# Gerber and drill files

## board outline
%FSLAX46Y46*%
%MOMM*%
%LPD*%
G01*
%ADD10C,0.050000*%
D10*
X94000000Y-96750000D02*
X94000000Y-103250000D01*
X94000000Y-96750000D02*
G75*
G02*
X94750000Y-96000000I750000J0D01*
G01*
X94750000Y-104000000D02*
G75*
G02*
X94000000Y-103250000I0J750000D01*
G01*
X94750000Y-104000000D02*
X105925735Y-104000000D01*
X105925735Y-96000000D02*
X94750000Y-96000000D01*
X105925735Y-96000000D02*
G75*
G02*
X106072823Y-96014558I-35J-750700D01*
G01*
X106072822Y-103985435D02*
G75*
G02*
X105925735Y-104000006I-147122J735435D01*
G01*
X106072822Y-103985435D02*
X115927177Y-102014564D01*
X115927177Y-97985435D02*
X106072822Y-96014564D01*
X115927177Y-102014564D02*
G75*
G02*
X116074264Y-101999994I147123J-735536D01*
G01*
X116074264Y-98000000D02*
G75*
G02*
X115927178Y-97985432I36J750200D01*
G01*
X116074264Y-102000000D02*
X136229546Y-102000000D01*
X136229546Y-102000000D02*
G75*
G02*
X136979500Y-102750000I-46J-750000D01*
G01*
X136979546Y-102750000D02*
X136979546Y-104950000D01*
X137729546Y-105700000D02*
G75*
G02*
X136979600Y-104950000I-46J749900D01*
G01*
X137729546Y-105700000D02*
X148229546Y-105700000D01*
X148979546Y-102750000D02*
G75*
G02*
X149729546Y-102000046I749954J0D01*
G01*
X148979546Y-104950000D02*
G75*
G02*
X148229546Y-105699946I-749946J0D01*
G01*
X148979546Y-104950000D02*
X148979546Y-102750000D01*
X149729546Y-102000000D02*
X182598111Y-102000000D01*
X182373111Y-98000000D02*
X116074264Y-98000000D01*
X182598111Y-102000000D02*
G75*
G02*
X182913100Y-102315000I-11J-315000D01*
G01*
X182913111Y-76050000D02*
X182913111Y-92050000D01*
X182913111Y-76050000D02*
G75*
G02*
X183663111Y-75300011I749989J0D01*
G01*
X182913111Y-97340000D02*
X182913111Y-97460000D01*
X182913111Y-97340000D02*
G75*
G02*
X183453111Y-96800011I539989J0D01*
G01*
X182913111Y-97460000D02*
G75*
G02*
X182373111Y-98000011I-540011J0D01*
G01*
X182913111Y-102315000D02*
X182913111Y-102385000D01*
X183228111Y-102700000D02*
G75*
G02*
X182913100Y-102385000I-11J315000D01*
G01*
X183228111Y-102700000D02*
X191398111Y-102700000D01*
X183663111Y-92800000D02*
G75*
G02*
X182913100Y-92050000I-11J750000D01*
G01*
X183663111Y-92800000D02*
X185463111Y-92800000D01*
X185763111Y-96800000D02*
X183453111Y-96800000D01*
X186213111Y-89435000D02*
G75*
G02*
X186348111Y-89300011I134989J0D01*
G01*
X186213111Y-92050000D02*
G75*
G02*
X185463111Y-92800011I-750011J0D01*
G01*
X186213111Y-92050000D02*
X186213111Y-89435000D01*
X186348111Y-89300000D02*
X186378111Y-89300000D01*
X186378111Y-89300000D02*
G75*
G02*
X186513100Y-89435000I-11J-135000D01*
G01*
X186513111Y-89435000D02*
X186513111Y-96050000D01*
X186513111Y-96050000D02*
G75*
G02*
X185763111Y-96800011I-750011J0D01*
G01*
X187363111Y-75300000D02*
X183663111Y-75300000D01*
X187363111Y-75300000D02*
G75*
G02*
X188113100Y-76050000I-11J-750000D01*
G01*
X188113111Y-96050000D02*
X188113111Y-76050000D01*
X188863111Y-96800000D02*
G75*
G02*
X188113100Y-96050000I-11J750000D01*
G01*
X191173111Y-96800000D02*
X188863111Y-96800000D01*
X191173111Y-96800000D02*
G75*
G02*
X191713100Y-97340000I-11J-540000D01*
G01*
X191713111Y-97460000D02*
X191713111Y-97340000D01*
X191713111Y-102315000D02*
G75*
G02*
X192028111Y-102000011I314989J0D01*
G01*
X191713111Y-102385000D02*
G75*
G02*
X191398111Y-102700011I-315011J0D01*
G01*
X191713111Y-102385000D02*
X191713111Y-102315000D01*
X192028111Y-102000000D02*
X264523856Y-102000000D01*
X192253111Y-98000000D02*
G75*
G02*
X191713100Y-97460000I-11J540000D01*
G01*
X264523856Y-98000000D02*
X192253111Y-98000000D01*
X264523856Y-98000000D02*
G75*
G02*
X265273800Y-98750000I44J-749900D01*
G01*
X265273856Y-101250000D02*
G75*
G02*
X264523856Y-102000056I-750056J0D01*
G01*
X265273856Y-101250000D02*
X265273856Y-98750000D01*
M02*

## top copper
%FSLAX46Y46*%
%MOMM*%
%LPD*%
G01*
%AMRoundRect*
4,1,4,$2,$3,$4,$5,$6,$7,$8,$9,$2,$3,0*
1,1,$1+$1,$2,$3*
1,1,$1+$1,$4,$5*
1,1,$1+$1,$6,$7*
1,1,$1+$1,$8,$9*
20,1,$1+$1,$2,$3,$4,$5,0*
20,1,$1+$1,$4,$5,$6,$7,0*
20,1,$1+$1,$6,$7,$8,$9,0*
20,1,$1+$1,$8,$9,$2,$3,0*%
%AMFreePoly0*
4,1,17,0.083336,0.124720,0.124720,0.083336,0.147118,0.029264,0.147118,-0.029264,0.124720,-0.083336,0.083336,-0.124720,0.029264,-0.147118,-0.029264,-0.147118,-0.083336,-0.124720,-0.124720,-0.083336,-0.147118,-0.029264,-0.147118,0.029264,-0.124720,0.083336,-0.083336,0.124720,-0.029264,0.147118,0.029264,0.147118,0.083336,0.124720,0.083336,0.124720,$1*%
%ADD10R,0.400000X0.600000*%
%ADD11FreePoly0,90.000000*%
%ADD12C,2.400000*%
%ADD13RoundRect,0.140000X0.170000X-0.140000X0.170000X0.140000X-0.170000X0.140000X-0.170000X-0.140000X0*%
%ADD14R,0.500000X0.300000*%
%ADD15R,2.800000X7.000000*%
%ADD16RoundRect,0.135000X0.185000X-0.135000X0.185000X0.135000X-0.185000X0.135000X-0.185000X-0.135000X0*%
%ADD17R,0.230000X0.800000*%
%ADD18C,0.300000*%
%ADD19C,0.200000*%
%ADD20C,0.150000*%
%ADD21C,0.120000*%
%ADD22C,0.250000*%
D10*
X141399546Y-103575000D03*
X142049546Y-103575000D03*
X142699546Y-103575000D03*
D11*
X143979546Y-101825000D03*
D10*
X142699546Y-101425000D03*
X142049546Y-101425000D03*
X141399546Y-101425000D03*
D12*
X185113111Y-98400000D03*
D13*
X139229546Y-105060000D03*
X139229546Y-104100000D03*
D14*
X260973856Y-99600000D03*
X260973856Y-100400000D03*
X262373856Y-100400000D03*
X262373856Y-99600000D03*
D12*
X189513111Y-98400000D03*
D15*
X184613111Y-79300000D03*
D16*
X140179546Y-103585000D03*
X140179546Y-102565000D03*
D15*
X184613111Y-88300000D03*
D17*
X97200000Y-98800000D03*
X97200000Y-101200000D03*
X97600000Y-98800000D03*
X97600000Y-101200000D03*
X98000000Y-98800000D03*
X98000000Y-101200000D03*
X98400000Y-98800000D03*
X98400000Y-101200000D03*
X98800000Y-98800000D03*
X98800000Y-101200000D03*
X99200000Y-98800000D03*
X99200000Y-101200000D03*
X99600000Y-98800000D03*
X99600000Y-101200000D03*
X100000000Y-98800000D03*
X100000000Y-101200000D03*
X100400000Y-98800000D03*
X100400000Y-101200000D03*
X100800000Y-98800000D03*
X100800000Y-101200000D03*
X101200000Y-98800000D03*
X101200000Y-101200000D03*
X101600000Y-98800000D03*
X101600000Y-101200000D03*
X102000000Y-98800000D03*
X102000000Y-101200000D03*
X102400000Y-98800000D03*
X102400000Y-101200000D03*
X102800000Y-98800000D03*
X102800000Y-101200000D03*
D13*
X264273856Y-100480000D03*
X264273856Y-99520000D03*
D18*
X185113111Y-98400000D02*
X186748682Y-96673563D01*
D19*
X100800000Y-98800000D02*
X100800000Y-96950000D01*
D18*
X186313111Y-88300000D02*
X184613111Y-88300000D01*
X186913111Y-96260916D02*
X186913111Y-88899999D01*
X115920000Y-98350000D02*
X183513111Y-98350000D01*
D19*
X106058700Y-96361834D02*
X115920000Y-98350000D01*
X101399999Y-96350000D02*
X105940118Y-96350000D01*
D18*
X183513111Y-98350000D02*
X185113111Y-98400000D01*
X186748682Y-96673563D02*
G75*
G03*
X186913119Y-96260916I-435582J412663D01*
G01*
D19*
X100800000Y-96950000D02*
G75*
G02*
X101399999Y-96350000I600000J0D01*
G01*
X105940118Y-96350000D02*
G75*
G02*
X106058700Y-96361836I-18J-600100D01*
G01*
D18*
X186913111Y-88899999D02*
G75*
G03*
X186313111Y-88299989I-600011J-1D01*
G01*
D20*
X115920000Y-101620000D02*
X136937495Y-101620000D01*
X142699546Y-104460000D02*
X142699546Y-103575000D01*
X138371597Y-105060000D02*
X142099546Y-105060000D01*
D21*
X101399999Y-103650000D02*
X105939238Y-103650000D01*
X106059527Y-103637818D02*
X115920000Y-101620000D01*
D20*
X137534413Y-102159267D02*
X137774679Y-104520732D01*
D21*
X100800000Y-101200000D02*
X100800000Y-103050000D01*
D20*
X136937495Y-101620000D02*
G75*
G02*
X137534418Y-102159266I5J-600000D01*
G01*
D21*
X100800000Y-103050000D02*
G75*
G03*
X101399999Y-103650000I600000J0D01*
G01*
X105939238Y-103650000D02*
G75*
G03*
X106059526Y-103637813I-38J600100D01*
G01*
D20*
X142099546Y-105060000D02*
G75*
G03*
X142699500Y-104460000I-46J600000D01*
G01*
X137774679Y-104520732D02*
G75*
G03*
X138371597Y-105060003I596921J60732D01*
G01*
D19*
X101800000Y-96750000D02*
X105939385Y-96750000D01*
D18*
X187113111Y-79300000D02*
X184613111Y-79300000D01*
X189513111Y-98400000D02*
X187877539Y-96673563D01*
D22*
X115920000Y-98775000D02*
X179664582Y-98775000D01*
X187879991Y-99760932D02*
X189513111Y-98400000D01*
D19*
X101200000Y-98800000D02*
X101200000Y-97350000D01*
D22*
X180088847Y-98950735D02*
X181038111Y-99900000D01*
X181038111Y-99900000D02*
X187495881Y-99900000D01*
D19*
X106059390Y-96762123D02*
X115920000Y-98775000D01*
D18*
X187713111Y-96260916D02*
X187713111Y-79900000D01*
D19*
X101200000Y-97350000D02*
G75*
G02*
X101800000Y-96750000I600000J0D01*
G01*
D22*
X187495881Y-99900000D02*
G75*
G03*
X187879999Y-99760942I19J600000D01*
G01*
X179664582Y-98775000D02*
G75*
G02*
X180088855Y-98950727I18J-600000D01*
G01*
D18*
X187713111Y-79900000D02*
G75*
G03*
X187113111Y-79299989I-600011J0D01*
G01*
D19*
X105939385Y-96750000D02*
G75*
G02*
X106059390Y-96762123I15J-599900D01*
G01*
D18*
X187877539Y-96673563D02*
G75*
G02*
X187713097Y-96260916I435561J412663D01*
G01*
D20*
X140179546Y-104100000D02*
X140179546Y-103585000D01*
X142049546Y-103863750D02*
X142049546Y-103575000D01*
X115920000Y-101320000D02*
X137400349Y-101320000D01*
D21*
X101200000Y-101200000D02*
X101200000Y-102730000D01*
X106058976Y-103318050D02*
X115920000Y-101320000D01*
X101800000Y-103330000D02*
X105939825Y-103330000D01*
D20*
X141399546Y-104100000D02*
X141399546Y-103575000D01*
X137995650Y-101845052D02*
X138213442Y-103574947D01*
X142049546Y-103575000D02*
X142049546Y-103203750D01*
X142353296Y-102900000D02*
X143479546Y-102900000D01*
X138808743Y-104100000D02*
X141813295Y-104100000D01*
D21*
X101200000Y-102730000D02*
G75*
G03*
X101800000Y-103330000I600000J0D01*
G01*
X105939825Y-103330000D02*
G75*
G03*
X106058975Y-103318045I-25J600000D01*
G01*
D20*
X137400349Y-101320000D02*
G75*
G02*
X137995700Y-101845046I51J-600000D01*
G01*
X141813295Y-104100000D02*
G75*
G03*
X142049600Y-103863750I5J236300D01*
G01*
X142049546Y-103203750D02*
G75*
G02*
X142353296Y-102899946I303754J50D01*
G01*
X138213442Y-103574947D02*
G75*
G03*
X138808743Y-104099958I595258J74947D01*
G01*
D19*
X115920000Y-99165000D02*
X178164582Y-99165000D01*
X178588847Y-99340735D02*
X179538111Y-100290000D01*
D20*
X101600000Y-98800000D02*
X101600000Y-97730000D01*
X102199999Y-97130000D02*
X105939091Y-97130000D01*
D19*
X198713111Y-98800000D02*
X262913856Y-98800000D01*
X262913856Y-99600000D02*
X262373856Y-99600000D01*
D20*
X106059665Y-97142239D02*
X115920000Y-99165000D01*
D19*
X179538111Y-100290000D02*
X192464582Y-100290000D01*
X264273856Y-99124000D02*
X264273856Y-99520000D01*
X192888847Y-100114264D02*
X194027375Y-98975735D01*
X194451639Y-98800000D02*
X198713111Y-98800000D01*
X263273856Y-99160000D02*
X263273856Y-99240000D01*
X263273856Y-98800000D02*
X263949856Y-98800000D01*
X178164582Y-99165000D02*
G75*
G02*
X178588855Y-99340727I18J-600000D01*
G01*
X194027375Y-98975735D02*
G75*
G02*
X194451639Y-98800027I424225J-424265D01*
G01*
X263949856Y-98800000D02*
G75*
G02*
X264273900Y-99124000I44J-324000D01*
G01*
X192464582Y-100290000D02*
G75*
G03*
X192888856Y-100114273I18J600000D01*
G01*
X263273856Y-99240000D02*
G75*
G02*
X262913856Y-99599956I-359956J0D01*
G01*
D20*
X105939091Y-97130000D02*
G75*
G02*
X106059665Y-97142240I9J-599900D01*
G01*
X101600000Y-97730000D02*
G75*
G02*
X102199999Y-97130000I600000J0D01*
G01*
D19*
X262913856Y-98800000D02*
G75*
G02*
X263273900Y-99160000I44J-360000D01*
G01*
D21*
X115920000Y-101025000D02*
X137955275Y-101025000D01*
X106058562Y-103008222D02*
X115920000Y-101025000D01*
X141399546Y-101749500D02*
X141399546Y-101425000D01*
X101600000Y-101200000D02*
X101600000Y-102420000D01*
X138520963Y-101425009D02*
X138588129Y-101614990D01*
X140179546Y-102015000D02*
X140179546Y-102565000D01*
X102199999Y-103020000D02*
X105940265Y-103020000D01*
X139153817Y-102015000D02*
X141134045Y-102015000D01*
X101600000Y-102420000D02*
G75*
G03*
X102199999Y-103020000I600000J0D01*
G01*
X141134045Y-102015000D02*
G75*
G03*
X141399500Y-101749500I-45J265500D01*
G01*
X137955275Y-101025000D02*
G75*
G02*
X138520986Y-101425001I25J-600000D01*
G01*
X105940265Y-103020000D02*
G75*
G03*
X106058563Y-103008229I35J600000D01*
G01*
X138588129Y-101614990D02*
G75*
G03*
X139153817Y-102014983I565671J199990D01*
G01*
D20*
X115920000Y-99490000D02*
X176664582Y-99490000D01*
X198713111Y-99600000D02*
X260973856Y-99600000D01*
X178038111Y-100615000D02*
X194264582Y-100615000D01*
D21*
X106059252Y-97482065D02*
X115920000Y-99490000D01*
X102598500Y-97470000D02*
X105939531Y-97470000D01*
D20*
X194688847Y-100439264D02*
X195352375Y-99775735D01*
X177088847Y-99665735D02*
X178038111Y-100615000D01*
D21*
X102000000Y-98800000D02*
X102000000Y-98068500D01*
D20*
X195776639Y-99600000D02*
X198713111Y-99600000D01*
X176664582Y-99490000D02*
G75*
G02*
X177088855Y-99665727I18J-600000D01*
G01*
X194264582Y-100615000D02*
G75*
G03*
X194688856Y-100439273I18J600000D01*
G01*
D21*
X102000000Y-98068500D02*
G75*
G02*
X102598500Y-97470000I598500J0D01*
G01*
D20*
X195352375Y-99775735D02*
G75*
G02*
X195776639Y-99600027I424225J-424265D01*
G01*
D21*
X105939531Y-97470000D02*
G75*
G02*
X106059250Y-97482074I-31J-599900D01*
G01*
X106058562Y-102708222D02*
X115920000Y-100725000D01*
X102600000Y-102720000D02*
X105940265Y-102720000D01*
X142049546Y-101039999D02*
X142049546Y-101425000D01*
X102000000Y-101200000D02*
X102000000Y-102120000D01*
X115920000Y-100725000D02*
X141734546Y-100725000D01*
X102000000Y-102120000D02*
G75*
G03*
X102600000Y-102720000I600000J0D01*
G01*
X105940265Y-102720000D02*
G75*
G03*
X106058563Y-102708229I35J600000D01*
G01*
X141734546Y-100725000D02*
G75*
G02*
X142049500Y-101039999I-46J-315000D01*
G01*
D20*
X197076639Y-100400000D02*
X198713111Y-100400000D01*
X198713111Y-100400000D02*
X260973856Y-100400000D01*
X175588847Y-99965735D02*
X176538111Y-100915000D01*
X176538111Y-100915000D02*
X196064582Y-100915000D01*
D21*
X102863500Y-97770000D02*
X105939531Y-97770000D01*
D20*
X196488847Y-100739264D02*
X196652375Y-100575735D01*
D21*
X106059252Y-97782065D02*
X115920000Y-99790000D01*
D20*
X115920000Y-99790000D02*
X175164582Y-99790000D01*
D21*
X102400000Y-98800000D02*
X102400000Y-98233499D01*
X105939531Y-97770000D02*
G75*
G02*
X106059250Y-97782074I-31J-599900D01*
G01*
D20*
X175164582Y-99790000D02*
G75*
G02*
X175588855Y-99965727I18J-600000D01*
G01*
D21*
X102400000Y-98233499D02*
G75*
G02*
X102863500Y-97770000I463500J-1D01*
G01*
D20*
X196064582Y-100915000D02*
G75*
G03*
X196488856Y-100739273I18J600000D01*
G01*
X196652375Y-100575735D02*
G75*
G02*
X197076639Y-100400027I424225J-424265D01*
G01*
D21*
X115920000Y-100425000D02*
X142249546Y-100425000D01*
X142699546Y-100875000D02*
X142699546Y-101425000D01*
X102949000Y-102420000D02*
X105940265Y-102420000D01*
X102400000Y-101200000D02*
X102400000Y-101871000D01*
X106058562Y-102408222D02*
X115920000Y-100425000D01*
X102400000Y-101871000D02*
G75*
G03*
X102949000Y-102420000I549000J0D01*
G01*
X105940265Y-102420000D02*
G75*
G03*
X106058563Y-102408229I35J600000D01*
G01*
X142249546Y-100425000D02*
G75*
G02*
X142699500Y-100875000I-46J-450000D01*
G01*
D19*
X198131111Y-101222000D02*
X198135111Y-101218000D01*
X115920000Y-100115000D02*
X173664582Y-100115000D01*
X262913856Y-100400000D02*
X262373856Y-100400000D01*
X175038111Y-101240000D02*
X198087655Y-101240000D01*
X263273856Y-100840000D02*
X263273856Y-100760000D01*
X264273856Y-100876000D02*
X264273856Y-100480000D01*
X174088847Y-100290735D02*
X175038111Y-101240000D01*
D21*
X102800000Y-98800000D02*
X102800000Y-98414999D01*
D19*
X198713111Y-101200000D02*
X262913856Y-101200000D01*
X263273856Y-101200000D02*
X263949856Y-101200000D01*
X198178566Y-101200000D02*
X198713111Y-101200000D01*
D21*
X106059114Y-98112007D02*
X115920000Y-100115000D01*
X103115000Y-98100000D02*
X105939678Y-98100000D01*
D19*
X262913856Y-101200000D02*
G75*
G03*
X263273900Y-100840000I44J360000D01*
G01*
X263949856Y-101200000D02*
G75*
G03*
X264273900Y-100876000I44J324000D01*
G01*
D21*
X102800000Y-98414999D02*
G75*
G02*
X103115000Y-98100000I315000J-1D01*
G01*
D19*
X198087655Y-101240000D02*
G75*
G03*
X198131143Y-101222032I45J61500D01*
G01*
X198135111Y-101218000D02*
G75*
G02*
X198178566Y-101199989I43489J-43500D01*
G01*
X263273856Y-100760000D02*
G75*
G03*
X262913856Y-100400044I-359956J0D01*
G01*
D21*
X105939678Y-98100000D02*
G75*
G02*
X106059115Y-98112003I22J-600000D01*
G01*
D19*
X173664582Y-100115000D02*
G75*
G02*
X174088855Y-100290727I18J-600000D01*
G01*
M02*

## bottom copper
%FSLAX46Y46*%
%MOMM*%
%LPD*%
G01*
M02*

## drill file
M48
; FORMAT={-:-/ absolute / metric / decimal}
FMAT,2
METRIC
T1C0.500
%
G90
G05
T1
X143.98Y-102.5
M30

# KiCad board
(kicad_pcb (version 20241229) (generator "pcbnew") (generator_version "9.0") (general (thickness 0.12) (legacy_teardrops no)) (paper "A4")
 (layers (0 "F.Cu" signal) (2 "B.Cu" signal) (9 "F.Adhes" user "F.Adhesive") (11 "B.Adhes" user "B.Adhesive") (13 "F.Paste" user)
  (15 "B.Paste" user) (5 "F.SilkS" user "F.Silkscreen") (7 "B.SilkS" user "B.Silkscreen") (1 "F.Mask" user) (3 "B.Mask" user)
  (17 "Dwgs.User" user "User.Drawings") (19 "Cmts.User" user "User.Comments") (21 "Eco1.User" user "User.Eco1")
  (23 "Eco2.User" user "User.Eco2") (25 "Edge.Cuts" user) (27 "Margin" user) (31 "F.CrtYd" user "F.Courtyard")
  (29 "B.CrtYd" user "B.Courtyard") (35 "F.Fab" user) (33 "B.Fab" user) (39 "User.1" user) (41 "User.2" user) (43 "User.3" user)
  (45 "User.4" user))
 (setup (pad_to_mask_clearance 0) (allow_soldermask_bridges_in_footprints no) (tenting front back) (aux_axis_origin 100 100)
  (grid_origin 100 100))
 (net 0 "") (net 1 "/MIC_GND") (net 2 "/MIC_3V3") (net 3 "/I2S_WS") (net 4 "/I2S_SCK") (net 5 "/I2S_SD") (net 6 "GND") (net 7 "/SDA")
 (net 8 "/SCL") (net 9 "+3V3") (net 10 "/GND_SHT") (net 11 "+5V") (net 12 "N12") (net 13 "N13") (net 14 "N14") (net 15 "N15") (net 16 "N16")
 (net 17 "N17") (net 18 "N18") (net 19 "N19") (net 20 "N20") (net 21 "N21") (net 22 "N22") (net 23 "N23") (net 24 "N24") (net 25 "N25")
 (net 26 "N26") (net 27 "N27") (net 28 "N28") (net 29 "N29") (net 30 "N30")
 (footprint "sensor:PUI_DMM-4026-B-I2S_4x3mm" (layer "F.Cu") (at 142.979546 102.5 90)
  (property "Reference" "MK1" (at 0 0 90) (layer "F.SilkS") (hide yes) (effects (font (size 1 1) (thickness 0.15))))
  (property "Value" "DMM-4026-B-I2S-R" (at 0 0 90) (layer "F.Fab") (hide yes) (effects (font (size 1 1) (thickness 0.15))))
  (pad "" np_thru_hole circle (at 0 1 90) (size 0.5 0.5) (drill 0.5) (layers "*.Mask"))
  (pad "1" smd rect (at -1.075 -1.58 90) (size 0.6 0.4) (layers "F.Cu" "F.Mask" "F.Paste") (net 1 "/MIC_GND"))
  (pad "2" smd rect (at -1.075 -0.93 90) (size 0.6 0.4) (layers "F.Cu" "F.Mask" "F.Paste") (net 1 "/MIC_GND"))
  (pad "3" smd rect (at -1.075 -0.28 90) (size 0.6 0.4) (layers "F.Cu" "F.Mask" "F.Paste") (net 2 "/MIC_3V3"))
  (pad "4" smd custom (at 0.675 1 90) (size 0.3 0.3) (layers "F.Cu" "F.Mask" "F.Paste") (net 1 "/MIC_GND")
   (options (clearance outline) (anchor circle)) (primitives))
  (pad "5" smd rect (at 1.075 -0.28 90) (size 0.6 0.4) (layers "F.Cu" "F.Mask" "F.Paste") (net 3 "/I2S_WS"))
  (pad "6" smd rect (at 1.075 -0.93 90) (size 0.6 0.4) (layers "F.Cu" "F.Mask" "F.Paste") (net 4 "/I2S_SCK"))
  (pad "7" smd rect (at 1.075 -1.58 90) (size 0.6 0.4) (layers "F.Cu" "F.Mask" "F.Paste") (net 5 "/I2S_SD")))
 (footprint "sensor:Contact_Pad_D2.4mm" (layer "F.Cu") (at 185.113111 98.4)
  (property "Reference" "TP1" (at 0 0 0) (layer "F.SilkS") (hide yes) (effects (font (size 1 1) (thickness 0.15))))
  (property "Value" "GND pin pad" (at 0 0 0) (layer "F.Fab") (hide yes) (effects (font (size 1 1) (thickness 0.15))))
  (pad "1" smd circle (at 0 0) (size 2.4 2.4) (layers "F.Cu" "F.Mask") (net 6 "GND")))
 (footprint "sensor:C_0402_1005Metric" (layer "F.Cu") (at 139.229546 104.58 90)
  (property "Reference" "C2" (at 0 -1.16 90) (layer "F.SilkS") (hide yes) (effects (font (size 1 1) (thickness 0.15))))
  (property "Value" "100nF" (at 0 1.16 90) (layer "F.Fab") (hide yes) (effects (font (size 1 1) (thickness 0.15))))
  (pad "1" smd roundrect (at -0.48 0 90) (size 0.56 0.62) (layers "F.Cu" "F.Mask" "F.Paste") (roundrect_rratio 0.25) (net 2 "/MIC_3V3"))
  (pad "2" smd roundrect (at 0.48 0 90) (size 0.56 0.62) (layers "F.Cu" "F.Mask" "F.Paste") (roundrect_rratio 0.25) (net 1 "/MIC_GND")))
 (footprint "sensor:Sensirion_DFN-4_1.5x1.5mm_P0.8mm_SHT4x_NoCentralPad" (layer "F.Cu") (at 261.673856 100)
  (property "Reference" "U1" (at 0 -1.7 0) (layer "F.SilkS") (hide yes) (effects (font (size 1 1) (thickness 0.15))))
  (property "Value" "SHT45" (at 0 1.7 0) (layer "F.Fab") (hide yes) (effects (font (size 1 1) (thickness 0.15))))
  (pad "1" smd rect (at -0.7 -0.4) (size 0.5 0.3) (layers "F.Cu" "F.Mask" "F.Paste") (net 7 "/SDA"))
  (pad "2" smd rect (at -0.7 0.4) (size 0.5 0.3) (layers "F.Cu" "F.Mask" "F.Paste") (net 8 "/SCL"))
  (pad "3" smd rect (at 0.7 0.4) (size 0.5 0.3) (layers "F.Cu" "F.Mask" "F.Paste") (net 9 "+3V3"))
  (pad "4" smd rect (at 0.7 -0.4) (size 0.5 0.3) (layers "F.Cu" "F.Mask" "F.Paste") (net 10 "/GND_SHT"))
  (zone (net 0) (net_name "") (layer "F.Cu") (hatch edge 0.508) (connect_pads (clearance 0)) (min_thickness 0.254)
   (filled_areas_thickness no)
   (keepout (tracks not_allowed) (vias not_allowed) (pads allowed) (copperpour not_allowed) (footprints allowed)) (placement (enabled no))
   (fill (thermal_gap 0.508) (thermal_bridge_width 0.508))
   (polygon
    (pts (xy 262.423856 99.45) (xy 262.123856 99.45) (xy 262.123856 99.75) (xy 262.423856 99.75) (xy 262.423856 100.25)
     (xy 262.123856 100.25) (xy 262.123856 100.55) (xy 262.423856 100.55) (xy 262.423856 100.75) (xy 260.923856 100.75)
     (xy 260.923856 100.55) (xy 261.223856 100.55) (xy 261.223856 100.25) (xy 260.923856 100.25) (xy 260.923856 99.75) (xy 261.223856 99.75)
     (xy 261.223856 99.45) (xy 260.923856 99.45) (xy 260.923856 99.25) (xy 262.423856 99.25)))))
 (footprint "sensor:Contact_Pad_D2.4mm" (layer "F.Cu") (at 189.513111 98.4)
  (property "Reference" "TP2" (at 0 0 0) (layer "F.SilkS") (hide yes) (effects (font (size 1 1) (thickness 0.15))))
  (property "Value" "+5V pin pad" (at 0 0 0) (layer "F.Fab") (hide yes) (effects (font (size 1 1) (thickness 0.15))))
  (pad "1" smd circle (at 0 0) (size 2.4 2.4) (layers "F.Cu" "F.Mask") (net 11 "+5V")))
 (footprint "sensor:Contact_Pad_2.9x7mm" (layer "F.Cu") (at 184.613111 79.3)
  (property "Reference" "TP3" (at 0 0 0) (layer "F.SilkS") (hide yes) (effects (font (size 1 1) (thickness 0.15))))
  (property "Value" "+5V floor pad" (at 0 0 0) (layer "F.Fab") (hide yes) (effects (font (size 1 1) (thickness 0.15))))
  (pad "1" smd rect (at 0 0) (size 2.8 7) (layers "F.Cu" "F.Mask") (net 11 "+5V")))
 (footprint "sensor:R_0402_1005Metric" (layer "F.Cu") (at 140.179546 103.075 90)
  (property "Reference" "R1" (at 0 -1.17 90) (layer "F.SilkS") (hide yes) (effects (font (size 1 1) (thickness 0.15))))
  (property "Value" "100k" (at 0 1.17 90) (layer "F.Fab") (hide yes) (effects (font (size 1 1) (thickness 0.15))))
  (pad "1" smd roundrect (at -0.51 0 90) (size 0.54 0.64) (layers "F.Cu" "F.Mask" "F.Paste") (roundrect_rratio 0.25) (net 1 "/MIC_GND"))
  (pad "2" smd roundrect (at 0.51 0 90) (size 0.54 0.64) (layers "F.Cu" "F.Mask" "F.Paste") (roundrect_rratio 0.25) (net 5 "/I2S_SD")))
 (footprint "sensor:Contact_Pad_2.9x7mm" (layer "F.Cu") (at 184.613111 88.3)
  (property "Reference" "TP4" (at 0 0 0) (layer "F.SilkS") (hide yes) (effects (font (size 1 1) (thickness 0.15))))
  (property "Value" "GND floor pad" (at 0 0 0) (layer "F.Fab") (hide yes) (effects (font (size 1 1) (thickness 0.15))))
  (pad "1" smd rect (at 0 0) (size 2.8 7) (layers "F.Cu" "F.Mask") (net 6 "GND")))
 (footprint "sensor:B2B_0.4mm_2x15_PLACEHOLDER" (layer "F.Cu") (at 100 100)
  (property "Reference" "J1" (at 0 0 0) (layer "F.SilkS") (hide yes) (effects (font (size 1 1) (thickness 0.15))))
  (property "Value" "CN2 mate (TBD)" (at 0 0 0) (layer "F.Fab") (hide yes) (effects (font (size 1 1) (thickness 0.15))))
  (pad "1" smd rect (at -2.8 -1.2) (size 0.23 0.8) (layers "F.Cu" "F.Mask" "F.Paste") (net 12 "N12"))
  (pad "2" smd rect (at -2.8 1.2) (size 0.23 0.8) (layers "F.Cu" "F.Mask" "F.Paste") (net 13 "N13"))
  (pad "3" smd rect (at -2.4 -1.2) (size 0.23 0.8) (layers "F.Cu" "F.Mask" "F.Paste") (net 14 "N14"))
  (pad "4" smd rect (at -2.4 1.2) (size 0.23 0.8) (layers "F.Cu" "F.Mask" "F.Paste") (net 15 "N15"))
  (pad "5" smd rect (at -2 -1.2) (size 0.23 0.8) (layers "F.Cu" "F.Mask" "F.Paste") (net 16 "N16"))
  (pad "6" smd rect (at -2 1.2) (size 0.23 0.8) (layers "F.Cu" "F.Mask" "F.Paste") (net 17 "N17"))
  (pad "7" smd rect (at -1.6 -1.2) (size 0.23 0.8) (layers "F.Cu" "F.Mask" "F.Paste") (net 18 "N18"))
  (pad "8" smd rect (at -1.6 1.2) (size 0.23 0.8) (layers "F.Cu" "F.Mask" "F.Paste") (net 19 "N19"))
  (pad "9" smd rect (at -1.2 -1.2) (size 0.23 0.8) (layers "F.Cu" "F.Mask" "F.Paste") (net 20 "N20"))
  (pad "10" smd rect (at -1.2 1.2) (size 0.23 0.8) (layers "F.Cu" "F.Mask" "F.Paste") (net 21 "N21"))
  (pad "11" smd rect (at -0.8 -1.2) (size 0.23 0.8) (layers "F.Cu" "F.Mask" "F.Paste") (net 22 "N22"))
  (pad "12" smd rect (at -0.8 1.2) (size 0.23 0.8) (layers "F.Cu" "F.Mask" "F.Paste") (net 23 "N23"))
  (pad "13" smd rect (at -0.4 -1.2) (size 0.23 0.8) (layers "F.Cu" "F.Mask" "F.Paste") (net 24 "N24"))
  (pad "14" smd rect (at -0.4 1.2) (size 0.23 0.8) (layers "F.Cu" "F.Mask" "F.Paste") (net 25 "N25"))
  (pad "15" smd rect (at 0 -1.2) (size 0.23 0.8) (layers "F.Cu" "F.Mask" "F.Paste") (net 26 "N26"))
  (pad "16" smd rect (at 0 1.2) (size 0.23 0.8) (layers "F.Cu" "F.Mask" "F.Paste") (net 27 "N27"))
  (pad "17" smd rect (at 0.4 -1.2) (size 0.23 0.8) (layers "F.Cu" "F.Mask" "F.Paste") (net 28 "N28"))
  (pad "18" smd rect (at 0.4 1.2) (size 0.23 0.8) (layers "F.Cu" "F.Mask" "F.Paste") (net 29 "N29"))
  (pad "19" smd rect (at 0.8 -1.2) (size 0.23 0.8) (layers "F.Cu" "F.Mask" "F.Paste") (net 6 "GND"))
  (pad "20" smd rect (at 0.8 1.2) (size 0.23 0.8) (layers "F.Cu" "F.Mask" "F.Paste") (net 2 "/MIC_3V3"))
  (pad "21" smd rect (at 1.2 -1.2) (size 0.23 0.8) (layers "F.Cu" "F.Mask" "F.Paste") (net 11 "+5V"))
  (pad "22" smd rect (at 1.2 1.2) (size 0.23 0.8) (layers "F.Cu" "F.Mask" "F.Paste") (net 1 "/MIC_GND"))
  (pad "23" smd rect (at 1.6 -1.2) (size 0.23 0.8) (layers "F.Cu" "F.Mask" "F.Paste") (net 10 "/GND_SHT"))
  (pad "24" smd rect (at 1.6 1.2) (size 0.23 0.8) (layers "F.Cu" "F.Mask" "F.Paste") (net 5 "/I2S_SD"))
  (pad "25" smd rect (at 2 -1.2) (size 0.23 0.8) (layers "F.Cu" "F.Mask" "F.Paste") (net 7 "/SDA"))
  (pad "26" smd rect (at 2 1.2) (size 0.23 0.8) (layers "F.Cu" "F.Mask" "F.Paste") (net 4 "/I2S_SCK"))
  (pad "27" smd rect (at 2.4 -1.2) (size 0.23 0.8) (layers "F.Cu" "F.Mask" "F.Paste") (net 8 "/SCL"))
  (pad "28" smd rect (at 2.4 1.2) (size 0.23 0.8) (layers "F.Cu" "F.Mask" "F.Paste") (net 3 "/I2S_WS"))
  (pad "29" smd rect (at 2.8 -1.2) (size 0.23 0.8) (layers "F.Cu" "F.Mask" "F.Paste") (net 9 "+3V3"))
  (pad "30" smd rect (at 2.8 1.2) (size 0.23 0.8) (layers "F.Cu" "F.Mask" "F.Paste") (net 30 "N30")))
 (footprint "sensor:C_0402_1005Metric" (layer "F.Cu") (at 264.273856 100 90)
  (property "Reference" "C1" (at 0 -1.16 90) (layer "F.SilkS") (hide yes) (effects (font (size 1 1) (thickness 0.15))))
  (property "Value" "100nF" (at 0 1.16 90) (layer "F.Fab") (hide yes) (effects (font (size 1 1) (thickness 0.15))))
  (pad "1" smd roundrect (at -0.48 0 90) (size 0.56 0.62) (layers "F.Cu" "F.Mask" "F.Paste") (roundrect_rratio 0.25) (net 9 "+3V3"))
  (pad "2" smd roundrect (at 0.48 0 90) (size 0.56 0.62) (layers "F.Cu" "F.Mask" "F.Paste") (roundrect_rratio 0.25) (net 10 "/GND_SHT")))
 (gr_line (start 94 96.75) (end 94 103.25) (stroke (width 0.05) (type default)) (layer "Edge.Cuts"))
 (gr_arc (start 94 96.75) (mid 94.21967 96.21967) (end 94.75 96) (stroke (width 0.05) (type default)) (layer "Edge.Cuts"))
 (gr_arc (start 94.75 104) (mid 94.21967 103.78033) (end 94 103.25) (stroke (width 0.05) (type default)) (layer "Edge.Cuts"))
 (gr_line (start 94.75 104) (end 105.925735 104) (stroke (width 0.05) (type default)) (layer "Edge.Cuts"))
 (gr_line (start 105.925735 96) (end 94.75 96) (stroke (width 0.05) (type default)) (layer "Edge.Cuts"))
 (gr_arc (start 105.925735 96) (mid 105.999638 96.003653) (end 106.072822 96.014564) (stroke (width 0.05) (type default))
  (layer "Edge.Cuts"))
 (gr_arc (start 106.072822 103.985435) (mid 105.999638 103.99635) (end 105.925735 104) (stroke (width 0.05) (type default))
  (layer "Edge.Cuts"))
 (gr_line (start 106.072822 103.985435) (end 115.927177 102.014564) (stroke (width 0.05) (type default)) (layer "Edge.Cuts"))
 (gr_line (start 115.927177 97.985435) (end 106.072822 96.014564) (stroke (width 0.05) (type default)) (layer "Edge.Cuts"))
 (gr_arc (start 115.927177 102.014564) (mid 116.000361 102.00365) (end 116.074264 102) (stroke (width 0.05) (type default))
  (layer "Edge.Cuts"))
 (gr_arc (start 116.074264 98) (mid 116.000361 97.996349) (end 115.927177 97.985435) (stroke (width 0.05) (type default))
  (layer "Edge.Cuts"))
 (gr_line (start 116.074264 102) (end 136.229546 102) (stroke (width 0.05) (type default)) (layer "Edge.Cuts"))
 (gr_arc (start 136.229546 102) (mid 136.759876 102.219669) (end 136.979546 102.75) (stroke (width 0.05) (type default)) (layer "Edge.Cuts"))
 (gr_line (start 136.979546 102.75) (end 136.979546 104.95) (stroke (width 0.05) (type default)) (layer "Edge.Cuts"))
 (gr_arc (start 137.729546 105.7) (mid 137.199186 105.480346) (end 136.979546 104.95) (stroke (width 0.05) (type default))
  (layer "Edge.Cuts"))
 (gr_line (start 137.729546 105.7) (end 148.229546 105.7) (stroke (width 0.05) (type default)) (layer "Edge.Cuts"))
 (gr_arc (start 148.979546 102.75) (mid 149.199216 102.219669) (end 149.729546 102) (stroke (width 0.05) (type default)) (layer "Edge.Cuts"))
 (gr_arc (start 148.979546 104.95) (mid 148.759879 105.480346) (end 148.229546 105.7) (stroke (width 0.05) (type default))
  (layer "Edge.Cuts"))
 (gr_line (start 148.979546 104.95) (end 148.979546 102.75) (stroke (width 0.05) (type default)) (layer "Edge.Cuts"))
 (gr_line (start 149.729546 102) (end 182.598111 102) (stroke (width 0.05) (type default)) (layer "Edge.Cuts"))
 (gr_line (start 182.373111 98) (end 116.074264 98) (stroke (width 0.05) (type default)) (layer "Edge.Cuts"))
 (gr_arc (start 182.598111 102) (mid 182.820849 102.092261) (end 182.913111 102.315) (stroke (width 0.05) (type default))
  (layer "Edge.Cuts"))
 (gr_line (start 182.913111 76.05) (end 182.913111 92.05) (stroke (width 0.05) (type default)) (layer "Edge.Cuts"))
 (gr_arc (start 182.913111 76.05) (mid 183.132782 75.519674) (end 183.663111 75.3) (stroke (width 0.05) (type default)) (layer "Edge.Cuts"))
 (gr_line (start 182.913111 97.34) (end 182.913111 97.46) (stroke (width 0.05) (type default)) (layer "Edge.Cuts"))
 (gr_arc (start 182.913111 97.34) (mid 183.071274 96.958166) (end 183.453111 96.8) (stroke (width 0.05) (type default)) (layer "Edge.Cuts"))
 (gr_arc (start 182.913111 97.46) (mid 182.754948 97.841837) (end 182.373111 98) (stroke (width 0.05) (type default)) (layer "Edge.Cuts"))
 (gr_line (start 182.913111 102.315) (end 182.913111 102.385) (stroke (width 0.05) (type default)) (layer "Edge.Cuts"))
 (gr_arc (start 183.228111 102.7) (mid 183.005365 102.607743) (end 182.913111 102.385) (stroke (width 0.05) (type default))
  (layer "Edge.Cuts"))
 (gr_line (start 183.228111 102.7) (end 191.398111 102.7) (stroke (width 0.05) (type default)) (layer "Edge.Cuts"))
 (gr_arc (start 183.663111 92.8) (mid 183.132774 92.580334) (end 182.913111 92.05) (stroke (width 0.05) (type default)) (layer "Edge.Cuts"))
 (gr_line (start 183.663111 92.8) (end 185.463111 92.8) (stroke (width 0.05) (type default)) (layer "Edge.Cuts"))
 (gr_line (start 185.763111 96.8) (end 183.453111 96.8) (stroke (width 0.05) (type default)) (layer "Edge.Cuts"))
 (gr_arc (start 186.213111 89.435) (mid 186.252651 89.33954) (end 186.348111 89.3) (stroke (width 0.05) (type default)) (layer "Edge.Cuts"))
 (gr_arc (start 186.213111 92.05) (mid 185.993442 92.580334) (end 185.463111 92.8) (stroke (width 0.05) (type default)) (layer "Edge.Cuts"))
 (gr_line (start 186.213111 92.05) (end 186.213111 89.435) (stroke (width 0.05) (type default)) (layer "Edge.Cuts"))
 (gr_line (start 186.348111 89.3) (end 186.378111 89.3) (stroke (width 0.05) (type default)) (layer "Edge.Cuts"))
 (gr_arc (start 186.378111 89.3) (mid 186.47357 89.33954) (end 186.513111 89.435) (stroke (width 0.05) (type default)) (layer "Edge.Cuts"))
 (gr_line (start 186.513111 89.435) (end 186.513111 96.05) (stroke (width 0.05) (type default)) (layer "Edge.Cuts"))
 (gr_arc (start 186.513111 96.05) (mid 186.293441 96.58033) (end 185.763111 96.8) (stroke (width 0.05) (type default)) (layer "Edge.Cuts"))
 (gr_line (start 187.363111 75.3) (end 183.663111 75.3) (stroke (width 0.05) (type default)) (layer "Edge.Cuts"))
 (gr_arc (start 187.363111 75.3) (mid 187.893434 75.519674) (end 188.113111 76.05) (stroke (width 0.05) (type default)) (layer "Edge.Cuts"))
 (gr_line (start 188.113111 96.05) (end 188.113111 76.05) (stroke (width 0.05) (type default)) (layer "Edge.Cuts"))
 (gr_arc (start 188.863111 96.8) (mid 188.332781 96.58033) (end 188.113111 96.05) (stroke (width 0.05) (type default)) (layer "Edge.Cuts"))
 (gr_line (start 191.173111 96.8) (end 188.863111 96.8) (stroke (width 0.05) (type default)) (layer "Edge.Cuts"))
 (gr_arc (start 191.173111 96.8) (mid 191.554942 96.958166) (end 191.713111 97.34) (stroke (width 0.05) (type default)) (layer "Edge.Cuts"))
 (gr_line (start 191.713111 97.46) (end 191.713111 97.34) (stroke (width 0.05) (type default)) (layer "Edge.Cuts"))
 (gr_arc (start 191.713111 102.315) (mid 191.805372 102.092261) (end 192.028111 102) (stroke (width 0.05) (type default))
  (layer "Edge.Cuts"))
 (gr_arc (start 191.713111 102.385) (mid 191.62085 102.607743) (end 191.398111 102.7) (stroke (width 0.05) (type default))
  (layer "Edge.Cuts"))
 (gr_line (start 191.713111 102.385) (end 191.713111 102.315) (stroke (width 0.05) (type default)) (layer "Edge.Cuts"))
 (gr_line (start 192.028111 102) (end 264.523856 102) (stroke (width 0.05) (type default)) (layer "Edge.Cuts"))
 (gr_arc (start 192.253111 98) (mid 191.871273 97.841837) (end 191.713111 97.46) (stroke (width 0.05) (type default)) (layer "Edge.Cuts"))
 (gr_line (start 264.523856 98) (end 192.253111 98) (stroke (width 0.05) (type default)) (layer "Edge.Cuts"))
 (gr_arc (start 264.523856 98) (mid 265.054215 98.219654) (end 265.273856 98.75) (stroke (width 0.05) (type default)) (layer "Edge.Cuts"))
 (gr_arc (start 265.273856 101.25) (mid 265.054183 101.780315) (end 264.523856 102) (stroke (width 0.05) (type default)) (layer "Edge.Cuts"))
 (gr_line (start 265.273856 101.25) (end 265.273856 98.75) (stroke (width 0.05) (type default)) (layer "Edge.Cuts"))
 (segment (start 185.113111 98.4) (end 186.748682 96.673563) (width 0.3) (layer "F.Cu") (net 6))
 (segment (start 100.8 98.8) (end 100.8 96.95) (width 0.2) (layer "F.Cu") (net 6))
 (segment (start 186.313111 88.3) (end 184.613111 88.3) (width 0.3) (layer "F.Cu") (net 6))
 (segment (start 186.913111 96.260916) (end 186.913111 88.899999) (width 0.3) (layer "F.Cu") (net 6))
 (segment (start 115.92 98.35) (end 183.513111 98.35) (width 0.3) (layer "F.Cu") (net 6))
 (segment (start 106.0587 96.361834) (end 115.92 98.35) (width 0.2) (layer "F.Cu") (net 6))
 (segment (start 101.399999 96.35) (end 105.940118 96.35) (width 0.2) (layer "F.Cu") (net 6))
 (segment (start 183.513111 98.35) (end 185.113111 98.4) (width 0.3) (layer "F.Cu") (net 6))
 (arc (start 186.748682 96.673563) (mid 186.87049 96.483016) (end 186.913111 96.260916) (width 0.3) (layer "F.Cu") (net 6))
 (arc (start 100.8 96.95) (mid 100.975735 96.525735) (end 101.399999 96.35) (width 0.2) (layer "F.Cu") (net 6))
 (arc (start 105.940118 96.35) (mid 105.999703 96.352966) (end 106.0587 96.361834) (width 0.2) (layer "F.Cu") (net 6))
 (arc (start 186.913111 88.899999) (mid 186.737375 88.475735) (end 186.313111 88.3) (width 0.3) (layer "F.Cu") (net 6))
 (segment (start 115.92 101.62) (end 136.937495 101.62) (width 0.15) (layer "F.Cu") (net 2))
 (segment (start 142.699546 104.46) (end 142.699546 103.575) (width 0.15) (layer "F.Cu") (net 2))
 (segment (start 138.371597 105.06) (end 142.099546 105.06) (width 0.15) (layer "F.Cu") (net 2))
 (segment (start 101.399999 103.65) (end 105.939238 103.65) (width 0.12) (layer "F.Cu") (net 2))
 (segment (start 106.059527 103.637818) (end 115.92 101.62) (width 0.12) (layer "F.Cu") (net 2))
 (segment (start 137.534413 102.159267) (end 137.774679 104.520732) (width 0.15) (layer "F.Cu") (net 2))
 (segment (start 100.8 101.2) (end 100.8 103.05) (width 0.12) (layer "F.Cu") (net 2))
 (arc (start 136.937495 101.62) (mid 137.339714 101.774781) (end 137.534413 102.159267) (width 0.15) (layer "F.Cu") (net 2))
 (arc (start 100.8 103.05) (mid 100.975735 103.474264) (end 101.399999 103.65) (width 0.12) (layer "F.Cu") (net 2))
 (arc (start 105.939238 103.65) (mid 105.99969 103.646946) (end 106.059527 103.637818) (width 0.12) (layer "F.Cu") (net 2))
 (arc (start 142.099546 105.06) (mid 142.52381 104.884264) (end 142.699546 104.46) (width 0.15) (layer "F.Cu") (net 2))
 (arc (start 137.774679 104.520732) (mid 137.969378 104.905218) (end 138.371597 105.06) (width 0.15) (layer "F.Cu") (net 2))
 (segment (start 101.8 96.75) (end 105.939385 96.75) (width 0.2) (layer "F.Cu") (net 11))
 (segment (start 187.113111 79.3) (end 184.613111 79.3) (width 0.3) (layer "F.Cu") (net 11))
 (segment (start 189.513111 98.4) (end 187.877539 96.673563) (width 0.3) (layer "F.Cu") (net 11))
 (segment (start 115.92 98.775) (end 179.664582 98.775) (width 0.25) (layer "F.Cu") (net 11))
 (segment (start 187.879991 99.760932) (end 189.513111 98.4) (width 0.25) (layer "F.Cu") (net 11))
 (segment (start 101.2 98.8) (end 101.2 97.35) (width 0.2) (layer "F.Cu") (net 11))
 (segment (start 180.088847 98.950735) (end 181.038111 99.9) (width 0.25) (layer "F.Cu") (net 11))
 (segment (start 181.038111 99.9) (end 187.495881 99.9) (width 0.25) (layer "F.Cu") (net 11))
 (segment (start 106.05939 96.762123) (end 115.92 98.775) (width 0.2) (layer "F.Cu") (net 11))
 (segment (start 187.713111 96.260916) (end 187.713111 79.9) (width 0.3) (layer "F.Cu") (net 11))
 (arc (start 101.2 97.35) (mid 101.375735 96.925735) (end 101.8 96.75) (width 0.2) (layer "F.Cu") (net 11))
 (arc (start 187.495881 99.9) (mid 187.700136 99.864162) (end 187.879991 99.760932) (width 0.25) (layer "F.Cu") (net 11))
 (arc (start 179.664582 98.775) (mid 179.894193 98.820672) (end 180.088847 98.950735) (width 0.25) (layer "F.Cu") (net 11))
 (arc (start 187.713111 79.9) (mid 187.537375 79.475735) (end 187.113111 79.3) (width 0.3) (layer "F.Cu") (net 11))
 (arc (start 105.939385 96.75) (mid 105.999693 96.753038) (end 106.05939 96.762123) (width 0.2) (layer "F.Cu") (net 11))
 (arc (start 187.877539 96.673563) (mid 187.755731 96.483016) (end 187.713111 96.260916) (width 0.3) (layer "F.Cu") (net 11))
 (segment (start 140.179546 104.1) (end 140.179546 103.585) (width 0.15) (layer "F.Cu") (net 1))
 (segment (start 142.049546 103.86375) (end 142.049546 103.575) (width 0.15) (layer "F.Cu") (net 1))
 (segment (start 115.92 101.32) (end 137.400349 101.32) (width 0.15) (layer "F.Cu") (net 1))
 (segment (start 101.2 101.2) (end 101.2 102.73) (width 0.12) (layer "F.Cu") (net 1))
 (segment (start 106.058976 103.31805) (end 115.92 101.32) (width 0.12) (layer "F.Cu") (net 1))
 (segment (start 101.8 103.33) (end 105.939825 103.33) (width 0.12) (layer "F.Cu") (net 1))
 (segment (start 141.399546 104.1) (end 141.399546 103.575) (width 0.15) (layer "F.Cu") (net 1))
 (segment (start 137.99565 101.845052) (end 138.213442 103.574947) (width 0.15) (layer "F.Cu") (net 1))
 (segment (start 142.049546 103.575) (end 142.049546 103.20375) (width 0.15) (layer "F.Cu") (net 1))
 (segment (start 142.353296 102.9) (end 143.479546 102.9) (width 0.15) (layer "F.Cu") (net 1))
 (segment (start 138.808743 104.1) (end 141.813295 104.1) (width 0.15) (layer "F.Cu") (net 1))
 (arc (start 101.2 102.73) (mid 101.375735 103.154264) (end 101.8 103.33) (width 0.12) (layer "F.Cu") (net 1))
 (arc (start 105.939825 103.33) (mid 105.999699 103.327005) (end 106.058976 103.31805) (width 0.12) (layer "F.Cu") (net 1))
 (arc (start 137.400349 101.32) (mid 137.797232 101.470017) (end 137.99565 101.845052) (width 0.15) (layer "F.Cu") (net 1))
 (arc (start 141.813295 104.1) (mid 141.980349 104.030803) (end 142.049546 103.86375) (width 0.15) (layer "F.Cu") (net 1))
 (arc (start 142.049546 103.20375) (mid 142.138512 102.988966) (end 142.353296 102.9) (width 0.15) (layer "F.Cu") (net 1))
 (arc (start 138.213442 103.574947) (mid 138.411861 103.949982) (end 138.808743 104.1) (width 0.15) (layer "F.Cu") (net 1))
 (segment (start 115.92 99.165) (end 178.164582 99.165) (width 0.2) (layer "F.Cu") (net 10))
 (segment (start 178.588847 99.340735) (end 179.538111 100.29) (width 0.2) (layer "F.Cu") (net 10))
 (segment (start 101.6 98.8) (end 101.6 97.73) (width 0.15) (layer "F.Cu") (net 10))
 (segment (start 102.199999 97.13) (end 105.939091 97.13) (width 0.15) (layer "F.Cu") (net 10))
 (segment (start 198.713111 98.8) (end 262.913856 98.8) (width 0.2) (layer "F.Cu") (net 10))
 (segment (start 262.913856 99.6) (end 262.373856 99.6) (width 0.2) (layer "F.Cu") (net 10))
 (segment (start 106.059665 97.142239) (end 115.92 99.165) (width 0.15) (layer "F.Cu") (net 10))
 (segment (start 179.538111 100.29) (end 192.464582 100.29) (width 0.2) (layer "F.Cu") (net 10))
 (segment (start 264.273856 99.124) (end 264.273856 99.52) (width 0.2) (layer "F.Cu") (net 10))
 (segment (start 192.888847 100.114264) (end 194.027375 98.975735) (width 0.2) (layer "F.Cu") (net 10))
 (segment (start 194.451639 98.8) (end 198.713111 98.8) (width 0.2) (layer "F.Cu") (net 10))
 (segment (start 263.273856 99.16) (end 263.273856 99.24) (width 0.2) (layer "F.Cu") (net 10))
 (segment (start 263.273856 98.8) (end 263.949856 98.8) (width 0.2) (layer "F.Cu") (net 10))
 (arc (start 178.164582 99.165) (mid 178.394193 99.210672) (end 178.588847 99.340735) (width 0.2) (layer "F.Cu") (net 10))
 (arc (start 194.027375 98.975735) (mid 194.222029 98.845672) (end 194.451639 98.8) (width 0.2) (layer "F.Cu") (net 10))
 (arc (start 263.949856 98.8) (mid 264.178958 98.894897) (end 264.273856 99.124) (width 0.2) (layer "F.Cu") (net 10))
 (arc (start 192.464582 100.29) (mid 192.694193 100.244327) (end 192.888847 100.114264) (width 0.2) (layer "F.Cu") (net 10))
 (arc (start 263.273856 99.24) (mid 263.168414 99.494558) (end 262.913856 99.6) (width 0.2) (layer "F.Cu") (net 10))
 (arc (start 105.939091 97.13) (mid 105.999688 97.133067) (end 106.059665 97.142239) (width 0.15) (layer "F.Cu") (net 10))
 (arc (start 101.6 97.73) (mid 101.775735 97.305735) (end 102.199999 97.13) (width 0.15) (layer "F.Cu") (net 10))
 (arc (start 262.913856 98.8) (mid 263.168414 98.905441) (end 263.273856 99.16) (width 0.2) (layer "F.Cu") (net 10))
 (segment (start 115.92 101.025) (end 137.955275 101.025) (width 0.12) (layer "F.Cu") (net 5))
 (segment (start 106.058562 103.008222) (end 115.92 101.025) (width 0.12) (layer "F.Cu") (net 5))
 (segment (start 141.399546 101.7495) (end 141.399546 101.425) (width 0.12) (layer "F.Cu") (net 5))
 (segment (start 101.6 101.2) (end 101.6 102.42) (width 0.12) (layer "F.Cu") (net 5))
 (segment (start 138.520963 101.425009) (end 138.588129 101.61499) (width 0.12) (layer "F.Cu") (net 5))
 (segment (start 140.179546 102.015) (end 140.179546 102.565) (width 0.12) (layer "F.Cu") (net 5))
 (segment (start 102.199999 103.02) (end 105.940265 103.02) (width 0.12) (layer "F.Cu") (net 5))
 (segment (start 139.153817 102.015) (end 141.134045 102.015) (width 0.12) (layer "F.Cu") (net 5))
 (arc (start 101.6 102.42) (mid 101.775735 102.844264) (end 102.199999 103.02) (width 0.12) (layer "F.Cu") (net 5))
 (arc (start 141.134045 102.015) (mid 141.321782 101.937236) (end 141.399546 101.7495) (width 0.12) (layer "F.Cu") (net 5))
 (arc (start 137.955275 101.025) (mid 138.301689 101.135104) (end 138.520963 101.425009) (width 0.12) (layer "F.Cu") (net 5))
 (arc (start 105.940265 103.02) (mid 105.999706 103.017048) (end 106.058562 103.008222) (width 0.12) (layer "F.Cu") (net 5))
 (arc (start 138.588129 101.61499) (mid 138.807403 101.904895) (end 139.153817 102.015) (width 0.12) (layer "F.Cu") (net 5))
 (segment (start 115.92 99.49) (end 176.664582 99.49) (width 0.15) (layer "F.Cu") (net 7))
 (segment (start 198.713111 99.6) (end 260.973856 99.6) (width 0.15) (layer "F.Cu") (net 7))
 (segment (start 178.038111 100.615) (end 194.264582 100.615) (width 0.15) (layer "F.Cu") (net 7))
 (segment (start 106.059252 97.482065) (end 115.92 99.49) (width 0.12) (layer "F.Cu") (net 7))
 (segment (start 102.5985 97.47) (end 105.939531 97.47) (width 0.12) (layer "F.Cu") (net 7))
 (segment (start 194.688847 100.439264) (end 195.352375 99.775735) (width 0.15) (layer "F.Cu") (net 7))
 (segment (start 177.088847 99.665735) (end 178.038111 100.615) (width 0.15) (layer "F.Cu") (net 7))
 (segment (start 102 98.8) (end 102 98.0685) (width 0.12) (layer "F.Cu") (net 7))
 (segment (start 195.776639 99.6) (end 198.713111 99.6) (width 0.15) (layer "F.Cu") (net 7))
 (arc (start 176.664582 99.49) (mid 176.894193 99.535672) (end 177.088847 99.665735) (width 0.15) (layer "F.Cu") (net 7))
 (arc (start 194.264582 100.615) (mid 194.494193 100.569327) (end 194.688847 100.439264) (width 0.15) (layer "F.Cu") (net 7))
 (arc (start 102 98.0685) (mid 102.175296 97.645296) (end 102.5985 97.47) (width 0.12) (layer "F.Cu") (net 7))
 (arc (start 195.352375 99.775735) (mid 195.547029 99.645672) (end 195.776639 99.6) (width 0.15) (layer "F.Cu") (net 7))
 (arc (start 105.939531 97.47) (mid 105.999695 97.473023) (end 106.059252 97.482065) (width 0.12) (layer "F.Cu") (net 7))
 (segment (start 106.058562 102.708222) (end 115.92 100.725) (width 0.12) (layer "F.Cu") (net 4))
 (segment (start 102.6 102.72) (end 105.940265 102.72) (width 0.12) (layer "F.Cu") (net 4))
 (segment (start 142.049546 101.039999) (end 142.049546 101.425) (width 0.12) (layer "F.Cu") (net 4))
 (segment (start 102 101.2) (end 102 102.12) (width 0.12) (layer "F.Cu") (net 4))
 (segment (start 115.92 100.725) (end 141.734546 100.725) (width 0.12) (layer "F.Cu") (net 4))
 (arc (start 102 102.12) (mid 102.175735 102.544264) (end 102.6 102.72) (width 0.12) (layer "F.Cu") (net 4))
 (arc (start 105.940265 102.72) (mid 105.999706 102.717048) (end 106.058562 102.708222) (width 0.12) (layer "F.Cu") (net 4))
 (arc (start 141.734546 100.725) (mid 141.957284 100.817261) (end 142.049546 101.039999) (width 0.12) (layer "F.Cu") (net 4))
 (segment (start 197.076639 100.4) (end 198.713111 100.4) (width 0.15) (layer "F.Cu") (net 8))
 (segment (start 198.713111 100.4) (end 260.973856 100.4) (width 0.15) (layer "F.Cu") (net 8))
 (segment (start 175.588847 99.965735) (end 176.538111 100.915) (width 0.15) (layer "F.Cu") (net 8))
 (segment (start 176.538111 100.915) (end 196.064582 100.915) (width 0.15) (layer "F.Cu") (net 8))
 (segment (start 102.8635 97.77) (end 105.939531 97.77) (width 0.12) (layer "F.Cu") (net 8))
 (segment (start 196.488847 100.739264) (end 196.652375 100.575735) (width 0.15) (layer "F.Cu") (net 8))
 (segment (start 106.059252 97.782065) (end 115.92 99.79) (width 0.12) (layer "F.Cu") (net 8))
 (segment (start 115.92 99.79) (end 175.164582 99.79) (width 0.15) (layer "F.Cu") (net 8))
 (segment (start 102.4 98.8) (end 102.4 98.233499) (width 0.12) (layer "F.Cu") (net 8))
 (arc (start 105.939531 97.77) (mid 105.999695 97.773023) (end 106.059252 97.782065) (width 0.12) (layer "F.Cu") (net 8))
 (arc (start 175.164582 99.79) (mid 175.394193 99.835672) (end 175.588847 99.965735) (width 0.15) (layer "F.Cu") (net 8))
 (arc (start 102.4 98.233499) (mid 102.535756 97.905756) (end 102.8635 97.77) (width 0.12) (layer "F.Cu") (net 8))
 (arc (start 196.064582 100.915) (mid 196.294193 100.869327) (end 196.488847 100.739264) (width 0.15) (layer "F.Cu") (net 8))
 (arc (start 196.652375 100.575735) (mid 196.847029 100.445672) (end 197.076639 100.4) (width 0.15) (layer "F.Cu") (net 8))
 (segment (start 115.92 100.425) (end 142.249546 100.425) (width 0.12) (layer "F.Cu") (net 3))
 (segment (start 142.699546 100.875) (end 142.699546 101.425) (width 0.12) (layer "F.Cu") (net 3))
 (segment (start 102.949 102.42) (end 105.940265 102.42) (width 0.12) (layer "F.Cu") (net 3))
 (segment (start 102.4 101.2) (end 102.4 101.871) (width 0.12) (layer "F.Cu") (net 3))
 (segment (start 106.058562 102.408222) (end 115.92 100.425) (width 0.12) (layer "F.Cu") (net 3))
 (arc (start 102.4 101.871) (mid 102.560798 102.259201) (end 102.949 102.42) (width 0.12) (layer "F.Cu") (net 3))
 (arc (start 105.940265 102.42) (mid 105.999706 102.417048) (end 106.058562 102.408222) (width 0.12) (layer "F.Cu") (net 3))
 (arc (start 142.249546 100.425) (mid 142.567744 100.556801) (end 142.699546 100.875) (width 0.12) (layer "F.Cu") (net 3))
 (segment (start 198.131111 101.222) (end 198.135111 101.218) (width 0.2) (layer "F.Cu") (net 9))
 (segment (start 115.92 100.115) (end 173.664582 100.115) (width 0.2) (layer "F.Cu") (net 9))
 (segment (start 262.913856 100.4) (end 262.373856 100.4) (width 0.2) (layer "F.Cu") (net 9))
 (segment (start 175.038111 101.24) (end 198.087655 101.24) (width 0.2) (layer "F.Cu") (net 9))
 (segment (start 263.273856 100.84) (end 263.273856 100.76) (width 0.2) (layer "F.Cu") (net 9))
 (segment (start 264.273856 100.876) (end 264.273856 100.48) (width 0.2) (layer "F.Cu") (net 9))
 (segment (start 174.088847 100.290735) (end 175.038111 101.24) (width 0.2) (layer "F.Cu") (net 9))
 (segment (start 102.8 98.8) (end 102.8 98.414999) (width 0.12) (layer "F.Cu") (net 9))
 (segment (start 198.713111 101.2) (end 262.913856 101.2) (width 0.2) (layer "F.Cu") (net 9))
 (segment (start 263.273856 101.2) (end 263.949856 101.2) (width 0.2) (layer "F.Cu") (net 9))
 (segment (start 198.178566 101.2) (end 198.713111 101.2) (width 0.2) (layer "F.Cu") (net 9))
 (segment (start 106.059114 98.112007) (end 115.92 100.115) (width 0.12) (layer "F.Cu") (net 9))
 (segment (start 103.115 98.1) (end 105.939678 98.1) (width 0.12) (layer "F.Cu") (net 9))
 (arc (start 262.913856 101.2) (mid 263.168414 101.094558) (end 263.273856 100.84) (width 0.2) (layer "F.Cu") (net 9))
 (arc (start 263.949856 101.2) (mid 264.178958 101.105102) (end 264.273856 100.876) (width 0.2) (layer "F.Cu") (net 9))
 (arc (start 102.8 98.414999) (mid 102.892261 98.192261) (end 103.115 98.1) (width 0.12) (layer "F.Cu") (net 9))
 (arc (start 198.087655 101.24) (mid 198.111173 101.235321) (end 198.131111 101.222) (width 0.2) (layer "F.Cu") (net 9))
 (arc (start 198.135111 101.218) (mid 198.155048 101.204678) (end 198.178566 101.2) (width 0.2) (layer "F.Cu") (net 9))
 (arc (start 263.273856 100.76) (mid 263.168414 100.505441) (end 262.913856 100.4) (width 0.2) (layer "F.Cu") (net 9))
 (arc (start 105.939678 98.1) (mid 105.999697 98.103009) (end 106.059114 98.112007) (width 0.12) (layer "F.Cu") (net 9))
 (arc (start 173.664582 100.115) (mid 173.894193 100.160672) (end 174.088847 100.290735) (width 0.2) (layer "F.Cu") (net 9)))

